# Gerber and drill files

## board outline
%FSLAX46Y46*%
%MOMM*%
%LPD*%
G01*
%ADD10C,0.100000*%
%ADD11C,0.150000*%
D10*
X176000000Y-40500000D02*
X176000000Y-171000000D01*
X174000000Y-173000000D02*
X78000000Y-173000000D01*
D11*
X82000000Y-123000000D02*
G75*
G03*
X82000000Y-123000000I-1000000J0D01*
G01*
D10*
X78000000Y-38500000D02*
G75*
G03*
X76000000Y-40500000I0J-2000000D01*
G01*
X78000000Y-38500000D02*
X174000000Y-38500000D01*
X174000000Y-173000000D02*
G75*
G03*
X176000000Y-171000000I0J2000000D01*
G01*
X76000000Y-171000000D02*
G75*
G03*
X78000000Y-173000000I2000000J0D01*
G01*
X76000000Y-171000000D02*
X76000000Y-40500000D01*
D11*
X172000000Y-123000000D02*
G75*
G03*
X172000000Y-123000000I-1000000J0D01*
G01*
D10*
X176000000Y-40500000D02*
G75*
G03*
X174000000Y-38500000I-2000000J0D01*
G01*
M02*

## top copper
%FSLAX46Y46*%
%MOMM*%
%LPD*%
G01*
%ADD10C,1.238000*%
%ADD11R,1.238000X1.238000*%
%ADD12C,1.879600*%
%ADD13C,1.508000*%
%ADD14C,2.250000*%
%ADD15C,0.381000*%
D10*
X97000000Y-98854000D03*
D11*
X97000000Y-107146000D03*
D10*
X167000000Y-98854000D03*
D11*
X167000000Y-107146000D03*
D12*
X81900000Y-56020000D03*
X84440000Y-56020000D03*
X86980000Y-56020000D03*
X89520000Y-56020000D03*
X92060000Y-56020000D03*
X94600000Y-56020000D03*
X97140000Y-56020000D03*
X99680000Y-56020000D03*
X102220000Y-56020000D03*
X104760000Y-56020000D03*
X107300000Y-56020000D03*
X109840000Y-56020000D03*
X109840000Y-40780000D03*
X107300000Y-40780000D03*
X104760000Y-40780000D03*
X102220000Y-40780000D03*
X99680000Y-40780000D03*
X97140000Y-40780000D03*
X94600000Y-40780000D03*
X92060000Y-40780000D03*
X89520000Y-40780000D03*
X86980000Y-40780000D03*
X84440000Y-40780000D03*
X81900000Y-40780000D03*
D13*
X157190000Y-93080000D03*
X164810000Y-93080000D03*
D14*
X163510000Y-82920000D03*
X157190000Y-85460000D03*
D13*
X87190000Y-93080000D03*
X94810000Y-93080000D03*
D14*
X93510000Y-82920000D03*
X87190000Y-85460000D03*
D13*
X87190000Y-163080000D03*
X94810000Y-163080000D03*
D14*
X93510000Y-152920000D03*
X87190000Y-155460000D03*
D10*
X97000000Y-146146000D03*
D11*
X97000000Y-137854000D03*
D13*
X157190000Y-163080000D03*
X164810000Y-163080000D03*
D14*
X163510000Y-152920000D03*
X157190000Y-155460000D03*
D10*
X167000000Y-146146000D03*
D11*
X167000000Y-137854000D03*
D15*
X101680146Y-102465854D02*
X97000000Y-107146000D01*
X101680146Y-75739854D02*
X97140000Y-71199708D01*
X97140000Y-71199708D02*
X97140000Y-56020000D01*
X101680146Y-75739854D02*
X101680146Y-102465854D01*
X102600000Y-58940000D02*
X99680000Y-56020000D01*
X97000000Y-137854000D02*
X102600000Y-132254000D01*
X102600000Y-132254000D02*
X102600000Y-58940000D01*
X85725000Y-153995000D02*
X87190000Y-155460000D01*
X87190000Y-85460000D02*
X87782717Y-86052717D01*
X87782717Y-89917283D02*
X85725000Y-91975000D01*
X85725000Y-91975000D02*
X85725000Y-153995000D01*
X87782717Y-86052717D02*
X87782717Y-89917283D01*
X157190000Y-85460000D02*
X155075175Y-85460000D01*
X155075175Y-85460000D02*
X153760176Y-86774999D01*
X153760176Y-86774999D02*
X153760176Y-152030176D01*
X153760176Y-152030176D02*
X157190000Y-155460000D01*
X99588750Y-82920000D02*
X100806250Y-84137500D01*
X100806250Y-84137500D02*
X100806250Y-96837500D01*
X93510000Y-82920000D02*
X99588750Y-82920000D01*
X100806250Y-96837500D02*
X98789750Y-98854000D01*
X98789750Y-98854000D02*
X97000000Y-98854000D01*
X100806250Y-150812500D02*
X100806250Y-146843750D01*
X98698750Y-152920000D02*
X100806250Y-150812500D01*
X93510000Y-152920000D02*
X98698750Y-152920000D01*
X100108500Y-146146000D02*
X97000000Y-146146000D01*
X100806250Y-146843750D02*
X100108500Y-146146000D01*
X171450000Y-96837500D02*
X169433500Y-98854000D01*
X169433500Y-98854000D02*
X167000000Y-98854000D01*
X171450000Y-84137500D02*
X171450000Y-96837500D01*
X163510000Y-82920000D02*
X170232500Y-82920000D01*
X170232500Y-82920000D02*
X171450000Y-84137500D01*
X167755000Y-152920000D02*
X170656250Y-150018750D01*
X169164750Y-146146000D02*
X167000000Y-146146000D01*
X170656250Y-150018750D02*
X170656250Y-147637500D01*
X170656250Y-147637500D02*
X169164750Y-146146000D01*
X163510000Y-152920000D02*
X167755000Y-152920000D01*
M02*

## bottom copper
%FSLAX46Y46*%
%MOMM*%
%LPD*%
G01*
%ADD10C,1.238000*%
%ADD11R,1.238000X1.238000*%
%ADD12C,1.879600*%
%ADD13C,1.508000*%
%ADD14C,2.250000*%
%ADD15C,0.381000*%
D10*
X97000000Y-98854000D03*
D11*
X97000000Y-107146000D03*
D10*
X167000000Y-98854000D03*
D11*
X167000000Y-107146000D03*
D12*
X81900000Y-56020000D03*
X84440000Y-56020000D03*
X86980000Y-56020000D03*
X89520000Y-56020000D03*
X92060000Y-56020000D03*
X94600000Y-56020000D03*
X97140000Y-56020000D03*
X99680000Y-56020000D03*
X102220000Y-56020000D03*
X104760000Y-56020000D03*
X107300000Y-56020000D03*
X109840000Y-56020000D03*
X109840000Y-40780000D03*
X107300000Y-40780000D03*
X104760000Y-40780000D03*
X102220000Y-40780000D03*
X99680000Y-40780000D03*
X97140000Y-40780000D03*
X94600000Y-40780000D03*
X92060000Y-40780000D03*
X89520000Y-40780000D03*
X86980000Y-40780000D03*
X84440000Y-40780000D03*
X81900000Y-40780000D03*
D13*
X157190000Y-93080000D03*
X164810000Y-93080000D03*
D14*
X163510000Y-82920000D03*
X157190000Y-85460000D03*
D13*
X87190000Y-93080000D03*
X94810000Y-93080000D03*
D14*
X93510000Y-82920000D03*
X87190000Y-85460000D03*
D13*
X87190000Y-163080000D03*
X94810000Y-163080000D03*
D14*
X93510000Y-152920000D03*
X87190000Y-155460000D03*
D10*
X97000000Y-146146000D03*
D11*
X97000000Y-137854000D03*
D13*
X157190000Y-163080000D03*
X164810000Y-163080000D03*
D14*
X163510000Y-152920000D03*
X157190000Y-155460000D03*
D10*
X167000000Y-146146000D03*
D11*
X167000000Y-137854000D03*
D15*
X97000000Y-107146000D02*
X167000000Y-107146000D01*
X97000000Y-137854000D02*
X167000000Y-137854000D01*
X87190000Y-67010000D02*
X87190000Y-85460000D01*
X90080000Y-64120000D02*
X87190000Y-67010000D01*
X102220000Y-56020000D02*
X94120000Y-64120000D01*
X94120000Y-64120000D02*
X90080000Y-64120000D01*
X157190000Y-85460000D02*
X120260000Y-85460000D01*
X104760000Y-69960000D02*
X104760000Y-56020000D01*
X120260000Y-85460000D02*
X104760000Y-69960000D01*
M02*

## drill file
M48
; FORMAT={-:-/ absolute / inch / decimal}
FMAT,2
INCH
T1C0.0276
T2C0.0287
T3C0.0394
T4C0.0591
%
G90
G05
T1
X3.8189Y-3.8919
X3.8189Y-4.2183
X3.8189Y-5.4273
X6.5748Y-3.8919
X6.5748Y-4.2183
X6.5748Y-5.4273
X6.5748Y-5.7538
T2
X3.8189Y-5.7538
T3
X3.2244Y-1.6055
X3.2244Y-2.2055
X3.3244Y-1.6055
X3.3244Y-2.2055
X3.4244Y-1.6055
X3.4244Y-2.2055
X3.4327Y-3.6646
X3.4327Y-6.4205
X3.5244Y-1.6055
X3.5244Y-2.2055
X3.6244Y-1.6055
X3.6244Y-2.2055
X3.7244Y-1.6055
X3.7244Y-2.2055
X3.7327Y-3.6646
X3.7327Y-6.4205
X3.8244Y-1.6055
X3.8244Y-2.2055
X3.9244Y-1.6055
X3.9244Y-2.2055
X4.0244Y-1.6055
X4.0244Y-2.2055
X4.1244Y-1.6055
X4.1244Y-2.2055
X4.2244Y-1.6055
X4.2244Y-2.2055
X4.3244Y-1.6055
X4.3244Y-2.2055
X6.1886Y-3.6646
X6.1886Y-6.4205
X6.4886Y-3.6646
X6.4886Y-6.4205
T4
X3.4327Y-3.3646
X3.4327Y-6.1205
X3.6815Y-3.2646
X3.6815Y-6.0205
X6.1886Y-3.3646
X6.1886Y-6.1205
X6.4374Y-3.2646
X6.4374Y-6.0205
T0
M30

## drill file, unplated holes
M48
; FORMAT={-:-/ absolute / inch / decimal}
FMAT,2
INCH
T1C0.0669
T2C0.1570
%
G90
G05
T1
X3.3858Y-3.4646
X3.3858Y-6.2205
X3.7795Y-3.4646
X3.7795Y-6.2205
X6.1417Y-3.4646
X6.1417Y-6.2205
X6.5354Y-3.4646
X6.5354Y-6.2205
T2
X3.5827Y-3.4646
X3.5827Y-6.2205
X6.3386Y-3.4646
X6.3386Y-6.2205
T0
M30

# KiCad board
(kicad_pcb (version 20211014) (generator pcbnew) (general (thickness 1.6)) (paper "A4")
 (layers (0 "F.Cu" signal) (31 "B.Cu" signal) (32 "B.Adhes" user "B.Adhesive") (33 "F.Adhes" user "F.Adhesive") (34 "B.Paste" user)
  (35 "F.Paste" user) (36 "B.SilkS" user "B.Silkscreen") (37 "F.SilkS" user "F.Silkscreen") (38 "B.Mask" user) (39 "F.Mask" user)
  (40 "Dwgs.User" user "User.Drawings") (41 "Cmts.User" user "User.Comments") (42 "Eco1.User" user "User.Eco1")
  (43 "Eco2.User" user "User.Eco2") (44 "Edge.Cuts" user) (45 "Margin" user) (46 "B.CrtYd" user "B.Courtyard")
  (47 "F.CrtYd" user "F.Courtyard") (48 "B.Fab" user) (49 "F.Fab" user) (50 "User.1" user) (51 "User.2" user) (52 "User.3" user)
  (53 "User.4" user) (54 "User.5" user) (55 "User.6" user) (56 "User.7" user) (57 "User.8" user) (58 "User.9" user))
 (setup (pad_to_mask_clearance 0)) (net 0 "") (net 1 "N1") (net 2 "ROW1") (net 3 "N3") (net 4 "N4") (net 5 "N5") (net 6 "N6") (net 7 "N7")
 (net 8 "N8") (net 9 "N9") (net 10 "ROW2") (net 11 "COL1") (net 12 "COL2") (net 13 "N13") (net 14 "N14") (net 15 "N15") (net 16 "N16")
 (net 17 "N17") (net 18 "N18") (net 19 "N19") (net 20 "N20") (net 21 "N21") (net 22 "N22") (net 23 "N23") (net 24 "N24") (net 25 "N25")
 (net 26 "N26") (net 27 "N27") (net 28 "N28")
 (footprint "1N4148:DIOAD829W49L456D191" (layer "F.Cu") (at 97 103 90)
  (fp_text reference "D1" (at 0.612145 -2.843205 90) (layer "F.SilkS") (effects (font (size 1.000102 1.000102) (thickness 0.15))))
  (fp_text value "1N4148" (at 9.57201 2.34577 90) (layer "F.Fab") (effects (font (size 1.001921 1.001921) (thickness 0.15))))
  (pad "A" thru_hole circle locked (at 4.146 0 90) (size 1.238 1.238) (drill 0.7) (layers *.Cu *.Mask) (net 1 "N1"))
  (pad "C" thru_hole rect locked (at -4.146 0 90) (size 1.238 1.238) (drill 0.7) (layers *.Cu *.Mask) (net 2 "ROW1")))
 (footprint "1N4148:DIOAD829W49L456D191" (layer "F.Cu") (at 167 103 90)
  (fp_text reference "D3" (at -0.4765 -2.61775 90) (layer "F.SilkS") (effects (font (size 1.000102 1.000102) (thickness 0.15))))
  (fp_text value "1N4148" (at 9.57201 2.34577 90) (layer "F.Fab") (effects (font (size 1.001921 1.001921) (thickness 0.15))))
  (pad "A" thru_hole circle locked (at 4.146 0 90) (size 1.238 1.238) (drill 0.7) (layers *.Cu *.Mask) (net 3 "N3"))
  (pad "C" thru_hole rect locked (at -4.146 0 90) (size 1.238 1.238) (drill 0.7) (layers *.Cu *.Mask) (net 2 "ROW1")))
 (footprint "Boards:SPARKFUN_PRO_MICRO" (layer "F.Cu") (at 94.6 48.4 90)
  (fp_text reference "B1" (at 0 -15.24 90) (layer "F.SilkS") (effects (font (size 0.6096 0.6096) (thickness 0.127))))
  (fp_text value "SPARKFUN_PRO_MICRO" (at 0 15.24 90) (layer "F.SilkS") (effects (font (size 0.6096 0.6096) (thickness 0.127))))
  (pad "1" thru_hole circle locked (at -7.62 -12.7 90) (size 1.8796 1.8796) (drill 1) (layers *.Cu *.Mask) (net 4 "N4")
   (solder_mask_margin 0.1016))
  (pad "2" thru_hole circle locked (at -7.62 -10.16 90) (size 1.8796 1.8796) (drill 1) (layers *.Cu *.Mask) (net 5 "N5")
   (solder_mask_margin 0.1016))
  (pad "3" thru_hole circle locked (at -7.62 -7.62 90) (size 1.8796 1.8796) (drill 1) (layers *.Cu *.Mask) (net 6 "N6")
   (solder_mask_margin 0.1016))
  (pad "4" thru_hole circle locked (at -7.62 -5.08 90) (size 1.8796 1.8796) (drill 1) (layers *.Cu *.Mask) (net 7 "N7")
   (solder_mask_margin 0.1016))
  (pad "5" thru_hole circle locked (at -7.62 -2.54 90) (size 1.8796 1.8796) (drill 1) (layers *.Cu *.Mask) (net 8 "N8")
   (solder_mask_margin 0.1016))
  (pad "6" thru_hole circle locked (at -7.62 0 90) (size 1.8796 1.8796) (drill 1) (layers *.Cu *.Mask) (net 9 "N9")
   (solder_mask_margin 0.1016))
  (pad "7" thru_hole circle locked (at -7.62 2.54 90) (size 1.8796 1.8796) (drill 1) (layers *.Cu *.Mask) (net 2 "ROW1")
   (solder_mask_margin 0.1016))
  (pad "8" thru_hole circle locked (at -7.62 5.08 90) (size 1.8796 1.8796) (drill 1) (layers *.Cu *.Mask) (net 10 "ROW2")
   (solder_mask_margin 0.1016))
  (pad "9" thru_hole circle locked (at -7.62 7.62 90) (size 1.8796 1.8796) (drill 1) (layers *.Cu *.Mask) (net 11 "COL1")
   (solder_mask_margin 0.1016))
  (pad "10" thru_hole circle locked (at -7.62 10.16 90) (size 1.8796 1.8796) (drill 1) (layers *.Cu *.Mask) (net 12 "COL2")
   (solder_mask_margin 0.1016))
  (pad "11" thru_hole circle locked (at -7.62 12.7 90) (size 1.8796 1.8796) (drill 1) (layers *.Cu *.Mask) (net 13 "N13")
   (solder_mask_margin 0.1016))
  (pad "12" thru_hole circle locked (at -7.62 15.24 90) (size 1.8796 1.8796) (drill 1) (layers *.Cu *.Mask) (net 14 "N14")
   (solder_mask_margin 0.1016))
  (pad "13" thru_hole circle locked (at 7.62 15.24 90) (size 1.8796 1.8796) (drill 1) (layers *.Cu *.Mask) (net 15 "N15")
   (solder_mask_margin 0.1016))
  (pad "14" thru_hole circle locked (at 7.62 12.7 90) (size 1.8796 1.8796) (drill 1) (layers *.Cu *.Mask) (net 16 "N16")
   (solder_mask_margin 0.1016))
  (pad "15" thru_hole circle locked (at 7.62 10.16 90) (size 1.8796 1.8796) (drill 1) (layers *.Cu *.Mask) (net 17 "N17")
   (solder_mask_margin 0.1016))
  (pad "16" thru_hole circle locked (at 7.62 7.62 90) (size 1.8796 1.8796) (drill 1) (layers *.Cu *.Mask) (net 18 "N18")
   (solder_mask_margin 0.1016))
  (pad "17" thru_hole circle locked (at 7.62 5.08 90) (size 1.8796 1.8796) (drill 1) (layers *.Cu *.Mask) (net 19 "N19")
   (solder_mask_margin 0.1016))
  (pad "18" thru_hole circle locked (at 7.62 2.54 90) (size 1.8796 1.8796) (drill 1) (layers *.Cu *.Mask) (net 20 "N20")
   (solder_mask_margin 0.1016))
  (pad "19" thru_hole circle locked (at 7.62 0 90) (size 1.8796 1.8796) (drill 1) (layers *.Cu *.Mask) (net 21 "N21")
   (solder_mask_margin 0.1016))
  (pad "20" thru_hole circle locked (at 7.62 -2.54 90) (size 1.8796 1.8796) (drill 1) (layers *.Cu *.Mask) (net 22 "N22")
   (solder_mask_margin 0.1016))
  (pad "21" thru_hole circle locked (at 7.62 -5.08 90) (size 1.8796 1.8796) (drill 1) (layers *.Cu *.Mask) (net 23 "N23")
   (solder_mask_margin 0.1016))
  (pad "22" thru_hole circle locked (at 7.62 -7.62 90) (size 1.8796 1.8796) (drill 1) (layers *.Cu *.Mask) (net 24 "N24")
   (solder_mask_margin 0.1016))
  (pad "23" thru_hole circle locked (at 7.62 -10.16 90) (size 1.8796 1.8796) (drill 1) (layers *.Cu *.Mask) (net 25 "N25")
   (solder_mask_margin 0.1016))
  (pad "24" thru_hole circle locked (at 7.62 -12.7 90) (size 1.8796 1.8796) (drill 1) (layers *.Cu *.Mask) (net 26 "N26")
   (solder_mask_margin 0.1016)))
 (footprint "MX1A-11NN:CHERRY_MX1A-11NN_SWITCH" (layer "F.Cu") (at 161 88)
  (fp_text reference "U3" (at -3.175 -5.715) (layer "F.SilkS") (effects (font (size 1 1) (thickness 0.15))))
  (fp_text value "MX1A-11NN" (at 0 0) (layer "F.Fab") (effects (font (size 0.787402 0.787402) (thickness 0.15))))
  (pad "" np_thru_hole circle locked (at 0 0) (size 3.9878 3.9878) (drill 3.9878) (layers *.Cu *.Mask))
  (pad "" np_thru_hole circle locked (at -5 0) (size 1.7 1.7) (drill 1.7) (layers *.Cu *.Mask))
  (pad "" np_thru_hole circle locked (at 5 0) (size 1.7 1.7) (drill 1.7) (layers *.Cu *.Mask))
  (pad "BR1" thru_hole circle locked (at -3.81 5.08) (size 1.508 1.508) (drill 1) (layers *.Cu *.Mask))
  (pad "BR2" thru_hole circle locked (at 3.81 5.08) (size 1.508 1.508) (drill 1) (layers *.Cu *.Mask))
  (pad "P$1" thru_hole circle locked (at 2.51 -5.08) (size 2.25 2.25) (drill 1.5) (layers *.Cu *.Mask) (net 3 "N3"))
  (pad "P$2" thru_hole circle locked (at -3.81 -2.54) (size 2.25 2.25) (drill 1.5) (layers *.Cu *.Mask) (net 12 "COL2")))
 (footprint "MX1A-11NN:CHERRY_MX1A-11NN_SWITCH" (layer "F.Cu") (at 91 88)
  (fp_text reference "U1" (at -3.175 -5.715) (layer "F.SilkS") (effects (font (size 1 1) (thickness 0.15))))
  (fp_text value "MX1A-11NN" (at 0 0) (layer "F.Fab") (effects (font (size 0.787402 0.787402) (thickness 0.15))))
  (pad "" np_thru_hole circle locked (at 5 0) (size 1.7 1.7) (drill 1.7) (layers *.Cu *.Mask))
  (pad "" np_thru_hole circle locked (at 0 0) (size 3.9878 3.9878) (drill 3.9878) (layers *.Cu *.Mask))
  (pad "" np_thru_hole circle locked (at -5 0) (size 1.7 1.7) (drill 1.7) (layers *.Cu *.Mask))
  (pad "BR1" thru_hole circle locked (at -3.81 5.08) (size 1.508 1.508) (drill 1) (layers *.Cu *.Mask))
  (pad "BR2" thru_hole circle locked (at 3.81 5.08) (size 1.508 1.508) (drill 1) (layers *.Cu *.Mask))
  (pad "P$1" thru_hole circle locked (at 2.51 -5.08) (size 2.25 2.25) (drill 1.5) (layers *.Cu *.Mask) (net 1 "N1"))
  (pad "P$2" thru_hole circle locked (at -3.81 -2.54) (size 2.25 2.25) (drill 1.5) (layers *.Cu *.Mask) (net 11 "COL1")))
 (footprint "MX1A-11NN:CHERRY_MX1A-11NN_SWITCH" (layer "F.Cu") (at 91 158)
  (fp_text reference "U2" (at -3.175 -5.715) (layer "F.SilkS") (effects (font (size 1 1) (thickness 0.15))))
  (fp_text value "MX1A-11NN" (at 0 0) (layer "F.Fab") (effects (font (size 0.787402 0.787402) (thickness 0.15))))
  (pad "" np_thru_hole circle locked (at -5 0) (size 1.7 1.7) (drill 1.7) (layers *.Cu *.Mask))
  (pad "" np_thru_hole circle locked (at 0 0) (size 3.9878 3.9878) (drill 3.9878) (layers *.Cu *.Mask))
  (pad "" np_thru_hole circle locked (at 5 0) (size 1.7 1.7) (drill 1.7) (layers *.Cu *.Mask))
  (pad "BR1" thru_hole circle locked (at -3.81 5.08) (size 1.508 1.508) (drill 1) (layers *.Cu *.Mask))
  (pad "BR2" thru_hole circle locked (at 3.81 5.08) (size 1.508 1.508) (drill 1) (layers *.Cu *.Mask))
  (pad "P$1" thru_hole circle locked (at 2.51 -5.08) (size 2.25 2.25) (drill 1.5) (layers *.Cu *.Mask) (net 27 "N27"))
  (pad "P$2" thru_hole circle locked (at -3.81 -2.54) (size 2.25 2.25) (drill 1.5) (layers *.Cu *.Mask) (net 11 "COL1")))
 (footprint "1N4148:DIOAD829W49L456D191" (layer "F.Cu") (at 97 142 -90)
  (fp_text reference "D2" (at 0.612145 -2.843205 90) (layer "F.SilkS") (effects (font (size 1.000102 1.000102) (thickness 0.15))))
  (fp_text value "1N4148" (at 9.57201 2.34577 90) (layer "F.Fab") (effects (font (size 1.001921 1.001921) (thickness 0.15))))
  (pad "A" thru_hole circle locked (at 4.146 0 270) (size 1.238 1.238) (drill 0.73) (layers *.Cu *.Mask) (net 27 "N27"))
  (pad "C" thru_hole rect locked (at -4.146 0 270) (size 1.238 1.238) (drill 0.7) (layers *.Cu *.Mask) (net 10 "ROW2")))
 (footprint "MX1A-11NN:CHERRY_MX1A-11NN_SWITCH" (layer "F.Cu") (at 161 158)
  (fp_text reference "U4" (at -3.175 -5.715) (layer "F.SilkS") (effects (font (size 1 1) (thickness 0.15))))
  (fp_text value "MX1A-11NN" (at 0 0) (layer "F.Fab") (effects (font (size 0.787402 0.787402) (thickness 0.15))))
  (pad "" np_thru_hole circle locked (at 5 0) (size 1.7 1.7) (drill 1.7) (layers *.Cu *.Mask))
  (pad "" np_thru_hole circle locked (at -5 0) (size 1.7 1.7) (drill 1.7) (layers *.Cu *.Mask))
  (pad "" np_thru_hole circle locked (at 0 0) (size 3.9878 3.9878) (drill 3.9878) (layers *.Cu *.Mask))
  (pad "BR1" thru_hole circle locked (at -3.81 5.08) (size 1.508 1.508) (drill 1) (layers *.Cu *.Mask))
  (pad "BR2" thru_hole circle locked (at 3.81 5.08) (size 1.508 1.508) (drill 1) (layers *.Cu *.Mask))
  (pad "P$1" thru_hole circle locked (at 2.51 -5.08) (size 2.25 2.25) (drill 1.5) (layers *.Cu *.Mask) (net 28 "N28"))
  (pad "P$2" thru_hole circle locked (at -3.81 -2.54) (size 2.25 2.25) (drill 1.5) (layers *.Cu *.Mask) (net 12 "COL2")))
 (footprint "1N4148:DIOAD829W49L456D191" (layer "F.Cu") (at 167 142 -90)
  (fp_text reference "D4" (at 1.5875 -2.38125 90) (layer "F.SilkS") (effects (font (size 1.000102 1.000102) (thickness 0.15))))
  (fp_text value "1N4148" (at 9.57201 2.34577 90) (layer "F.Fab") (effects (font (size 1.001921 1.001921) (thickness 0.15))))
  (pad "A" thru_hole circle locked (at 4.146 0 270) (size 1.238 1.238) (drill 0.7) (layers *.Cu *.Mask) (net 28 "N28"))
  (pad "C" thru_hole rect locked (at -4.146 0 270) (size 1.238 1.238) (drill 0.7) (layers *.Cu *.Mask) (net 10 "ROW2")))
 (gr_line (start 176 40.5) (end 176 171) (layer "Edge.Cuts") (width 0.1))
 (gr_line (start 174 173) (end 78 173) (layer "Edge.Cuts") (width 0.1))
 (gr_circle (center 81 123) (end 82 123) (layer "Edge.Cuts") (width 0.15) (fill none))
 (gr_arc (start 76 40.5) (mid 76.585786 39.085786) (end 78 38.5) (layer "Edge.Cuts") (width 0.1))
 (gr_line (start 78 38.5) (end 174 38.5) (layer "Edge.Cuts") (width 0.1))
 (gr_arc (start 176 171) (mid 175.414214 172.414214) (end 174 173) (layer "Edge.Cuts") (width 0.1))
 (gr_arc (start 78 173) (mid 76.585786 172.414214) (end 76 171) (layer "Edge.Cuts") (width 0.1))
 (gr_line (start 76 171) (end 76 40.5) (layer "Edge.Cuts") (width 0.1))
 (gr_circle (center 171 123) (end 172 123) (layer "Edge.Cuts") (width 0.15) (fill none))
 (gr_arc (start 174 38.5) (mid 175.414214 39.085786) (end 176 40.5) (layer "Edge.Cuts") (width 0.1))
 (segment (start 101.680146 102.465854) (end 97 107.146) (width 0.381) (layer "F.Cu") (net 2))
 (segment (start 101.680146 75.739854) (end 97.14 71.199708) (width 0.381) (layer "F.Cu") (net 2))
 (segment (start 97.14 71.199708) (end 97.14 56.02) (width 0.381) (layer "F.Cu") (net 2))
 (segment (start 101.680146 75.739854) (end 101.680146 102.465854) (width 0.381) (layer "F.Cu") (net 2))
 (segment (start 97 107.146) (end 167 107.146) (width 0.381) (layer "B.Cu") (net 2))
 (segment (start 102.6 58.94) (end 99.68 56.02) (width 0.381) (layer "F.Cu") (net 10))
 (segment (start 97 137.854) (end 102.6 132.254) (width 0.381) (layer "F.Cu") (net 10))
 (segment (start 102.6 132.254) (end 102.6 58.94) (width 0.381) (layer "F.Cu") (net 10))
 (segment (start 97 137.854) (end 167 137.854) (width 0.381) (layer "B.Cu") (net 10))
 (segment (start 85.725 153.995) (end 87.19 155.46) (width 0.381) (layer "F.Cu") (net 11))
 (segment (start 87.19 85.46) (end 87.782717 86.052717) (width 0.381) (layer "F.Cu") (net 11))
 (segment (start 87.782717 89.917283) (end 85.725 91.975) (width 0.381) (layer "F.Cu") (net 11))
 (segment (start 85.725 91.975) (end 85.725 153.995) (width 0.381) (layer "F.Cu") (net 11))
 (segment (start 87.782717 86.052717) (end 87.782717 89.917283) (width 0.381) (layer "F.Cu") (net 11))
 (segment (start 87.19 67.01) (end 87.19 85.46) (width 0.381) (layer "B.Cu") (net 11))
 (segment (start 90.08 64.12) (end 87.19 67.01) (width 0.381) (layer "B.Cu") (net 11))
 (segment (start 102.22 56.02) (end 94.12 64.12) (width 0.381) (layer "B.Cu") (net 11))
 (segment (start 94.12 64.12) (end 90.08 64.12) (width 0.381) (layer "B.Cu") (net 11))
 (segment (start 157.19 85.46) (end 155.075175 85.46) (width 0.381) (layer "F.Cu") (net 12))
 (segment (start 155.075175 85.46) (end 153.760176 86.774999) (width 0.381) (layer "F.Cu") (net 12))
 (segment (start 153.760176 86.774999) (end 153.760176 152.030176) (width 0.381) (layer "F.Cu") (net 12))
 (segment (start 153.760176 152.030176) (end 157.19 155.46) (width 0.381) (layer "F.Cu") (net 12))
 (segment (start 157.19 85.46) (end 120.26 85.46) (width 0.381) (layer "B.Cu") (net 12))
 (segment (start 104.76 69.96) (end 104.76 56.02) (width 0.381) (layer "B.Cu") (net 12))
 (segment (start 120.26 85.46) (end 104.76 69.96) (width 0.381) (layer "B.Cu") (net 12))
 (segment (start 99.58875 82.92) (end 100.80625 84.1375) (width 0.381) (layer "F.Cu") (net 1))
 (segment (start 100.80625 84.1375) (end 100.80625 96.8375) (width 0.381) (layer "F.Cu") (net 1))
 (segment (start 93.51 82.92) (end 99.58875 82.92) (width 0.381) (layer "F.Cu") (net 1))
 (segment (start 100.80625 96.8375) (end 98.78975 98.854) (width 0.381) (layer "F.Cu") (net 1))
 (segment (start 98.78975 98.854) (end 97 98.854) (width 0.381) (layer "F.Cu") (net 1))
 (segment (start 100.80625 150.8125) (end 100.80625 146.84375) (width 0.381) (layer "F.Cu") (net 27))
 (segment (start 98.69875 152.92) (end 100.80625 150.8125) (width 0.381) (layer "F.Cu") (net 27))
 (segment (start 93.51 152.92) (end 98.69875 152.92) (width 0.381) (layer "F.Cu") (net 27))
 (segment (start 100.1085 146.146) (end 97 146.146) (width 0.381) (layer "F.Cu") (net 27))
 (segment (start 100.80625 146.84375) (end 100.1085 146.146) (width 0.381) (layer "F.Cu") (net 27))
 (segment (start 171.45 96.8375) (end 169.4335 98.854) (width 0.381) (layer "F.Cu") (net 3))
 (segment (start 169.4335 98.854) (end 167 98.854) (width 0.381) (layer "F.Cu") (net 3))
 (segment (start 171.45 84.1375) (end 171.45 96.8375) (width 0.381) (layer "F.Cu") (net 3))
 (segment (start 163.51 82.92) (end 170.2325 82.92) (width 0.381) (layer "F.Cu") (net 3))
 (segment (start 170.2325 82.92) (end 171.45 84.1375) (width 0.381) (layer "F.Cu") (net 3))
 (segment (start 167.755 152.92) (end 170.65625 150.01875) (width 0.381) (layer "F.Cu") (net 28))
 (segment (start 169.16475 146.146) (end 167 146.146) (width 0.381) (layer "F.Cu") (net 28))
 (segment (start 170.65625 150.01875) (end 170.65625 147.6375) (width 0.381) (layer "F.Cu") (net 28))
 (segment (start 170.65625 147.6375) (end 169.16475 146.146) (width 0.381) (layer "F.Cu") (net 28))
 (segment (start 163.51 152.92) (end 167.755 152.92) (width 0.381) (layer "F.Cu") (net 28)))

